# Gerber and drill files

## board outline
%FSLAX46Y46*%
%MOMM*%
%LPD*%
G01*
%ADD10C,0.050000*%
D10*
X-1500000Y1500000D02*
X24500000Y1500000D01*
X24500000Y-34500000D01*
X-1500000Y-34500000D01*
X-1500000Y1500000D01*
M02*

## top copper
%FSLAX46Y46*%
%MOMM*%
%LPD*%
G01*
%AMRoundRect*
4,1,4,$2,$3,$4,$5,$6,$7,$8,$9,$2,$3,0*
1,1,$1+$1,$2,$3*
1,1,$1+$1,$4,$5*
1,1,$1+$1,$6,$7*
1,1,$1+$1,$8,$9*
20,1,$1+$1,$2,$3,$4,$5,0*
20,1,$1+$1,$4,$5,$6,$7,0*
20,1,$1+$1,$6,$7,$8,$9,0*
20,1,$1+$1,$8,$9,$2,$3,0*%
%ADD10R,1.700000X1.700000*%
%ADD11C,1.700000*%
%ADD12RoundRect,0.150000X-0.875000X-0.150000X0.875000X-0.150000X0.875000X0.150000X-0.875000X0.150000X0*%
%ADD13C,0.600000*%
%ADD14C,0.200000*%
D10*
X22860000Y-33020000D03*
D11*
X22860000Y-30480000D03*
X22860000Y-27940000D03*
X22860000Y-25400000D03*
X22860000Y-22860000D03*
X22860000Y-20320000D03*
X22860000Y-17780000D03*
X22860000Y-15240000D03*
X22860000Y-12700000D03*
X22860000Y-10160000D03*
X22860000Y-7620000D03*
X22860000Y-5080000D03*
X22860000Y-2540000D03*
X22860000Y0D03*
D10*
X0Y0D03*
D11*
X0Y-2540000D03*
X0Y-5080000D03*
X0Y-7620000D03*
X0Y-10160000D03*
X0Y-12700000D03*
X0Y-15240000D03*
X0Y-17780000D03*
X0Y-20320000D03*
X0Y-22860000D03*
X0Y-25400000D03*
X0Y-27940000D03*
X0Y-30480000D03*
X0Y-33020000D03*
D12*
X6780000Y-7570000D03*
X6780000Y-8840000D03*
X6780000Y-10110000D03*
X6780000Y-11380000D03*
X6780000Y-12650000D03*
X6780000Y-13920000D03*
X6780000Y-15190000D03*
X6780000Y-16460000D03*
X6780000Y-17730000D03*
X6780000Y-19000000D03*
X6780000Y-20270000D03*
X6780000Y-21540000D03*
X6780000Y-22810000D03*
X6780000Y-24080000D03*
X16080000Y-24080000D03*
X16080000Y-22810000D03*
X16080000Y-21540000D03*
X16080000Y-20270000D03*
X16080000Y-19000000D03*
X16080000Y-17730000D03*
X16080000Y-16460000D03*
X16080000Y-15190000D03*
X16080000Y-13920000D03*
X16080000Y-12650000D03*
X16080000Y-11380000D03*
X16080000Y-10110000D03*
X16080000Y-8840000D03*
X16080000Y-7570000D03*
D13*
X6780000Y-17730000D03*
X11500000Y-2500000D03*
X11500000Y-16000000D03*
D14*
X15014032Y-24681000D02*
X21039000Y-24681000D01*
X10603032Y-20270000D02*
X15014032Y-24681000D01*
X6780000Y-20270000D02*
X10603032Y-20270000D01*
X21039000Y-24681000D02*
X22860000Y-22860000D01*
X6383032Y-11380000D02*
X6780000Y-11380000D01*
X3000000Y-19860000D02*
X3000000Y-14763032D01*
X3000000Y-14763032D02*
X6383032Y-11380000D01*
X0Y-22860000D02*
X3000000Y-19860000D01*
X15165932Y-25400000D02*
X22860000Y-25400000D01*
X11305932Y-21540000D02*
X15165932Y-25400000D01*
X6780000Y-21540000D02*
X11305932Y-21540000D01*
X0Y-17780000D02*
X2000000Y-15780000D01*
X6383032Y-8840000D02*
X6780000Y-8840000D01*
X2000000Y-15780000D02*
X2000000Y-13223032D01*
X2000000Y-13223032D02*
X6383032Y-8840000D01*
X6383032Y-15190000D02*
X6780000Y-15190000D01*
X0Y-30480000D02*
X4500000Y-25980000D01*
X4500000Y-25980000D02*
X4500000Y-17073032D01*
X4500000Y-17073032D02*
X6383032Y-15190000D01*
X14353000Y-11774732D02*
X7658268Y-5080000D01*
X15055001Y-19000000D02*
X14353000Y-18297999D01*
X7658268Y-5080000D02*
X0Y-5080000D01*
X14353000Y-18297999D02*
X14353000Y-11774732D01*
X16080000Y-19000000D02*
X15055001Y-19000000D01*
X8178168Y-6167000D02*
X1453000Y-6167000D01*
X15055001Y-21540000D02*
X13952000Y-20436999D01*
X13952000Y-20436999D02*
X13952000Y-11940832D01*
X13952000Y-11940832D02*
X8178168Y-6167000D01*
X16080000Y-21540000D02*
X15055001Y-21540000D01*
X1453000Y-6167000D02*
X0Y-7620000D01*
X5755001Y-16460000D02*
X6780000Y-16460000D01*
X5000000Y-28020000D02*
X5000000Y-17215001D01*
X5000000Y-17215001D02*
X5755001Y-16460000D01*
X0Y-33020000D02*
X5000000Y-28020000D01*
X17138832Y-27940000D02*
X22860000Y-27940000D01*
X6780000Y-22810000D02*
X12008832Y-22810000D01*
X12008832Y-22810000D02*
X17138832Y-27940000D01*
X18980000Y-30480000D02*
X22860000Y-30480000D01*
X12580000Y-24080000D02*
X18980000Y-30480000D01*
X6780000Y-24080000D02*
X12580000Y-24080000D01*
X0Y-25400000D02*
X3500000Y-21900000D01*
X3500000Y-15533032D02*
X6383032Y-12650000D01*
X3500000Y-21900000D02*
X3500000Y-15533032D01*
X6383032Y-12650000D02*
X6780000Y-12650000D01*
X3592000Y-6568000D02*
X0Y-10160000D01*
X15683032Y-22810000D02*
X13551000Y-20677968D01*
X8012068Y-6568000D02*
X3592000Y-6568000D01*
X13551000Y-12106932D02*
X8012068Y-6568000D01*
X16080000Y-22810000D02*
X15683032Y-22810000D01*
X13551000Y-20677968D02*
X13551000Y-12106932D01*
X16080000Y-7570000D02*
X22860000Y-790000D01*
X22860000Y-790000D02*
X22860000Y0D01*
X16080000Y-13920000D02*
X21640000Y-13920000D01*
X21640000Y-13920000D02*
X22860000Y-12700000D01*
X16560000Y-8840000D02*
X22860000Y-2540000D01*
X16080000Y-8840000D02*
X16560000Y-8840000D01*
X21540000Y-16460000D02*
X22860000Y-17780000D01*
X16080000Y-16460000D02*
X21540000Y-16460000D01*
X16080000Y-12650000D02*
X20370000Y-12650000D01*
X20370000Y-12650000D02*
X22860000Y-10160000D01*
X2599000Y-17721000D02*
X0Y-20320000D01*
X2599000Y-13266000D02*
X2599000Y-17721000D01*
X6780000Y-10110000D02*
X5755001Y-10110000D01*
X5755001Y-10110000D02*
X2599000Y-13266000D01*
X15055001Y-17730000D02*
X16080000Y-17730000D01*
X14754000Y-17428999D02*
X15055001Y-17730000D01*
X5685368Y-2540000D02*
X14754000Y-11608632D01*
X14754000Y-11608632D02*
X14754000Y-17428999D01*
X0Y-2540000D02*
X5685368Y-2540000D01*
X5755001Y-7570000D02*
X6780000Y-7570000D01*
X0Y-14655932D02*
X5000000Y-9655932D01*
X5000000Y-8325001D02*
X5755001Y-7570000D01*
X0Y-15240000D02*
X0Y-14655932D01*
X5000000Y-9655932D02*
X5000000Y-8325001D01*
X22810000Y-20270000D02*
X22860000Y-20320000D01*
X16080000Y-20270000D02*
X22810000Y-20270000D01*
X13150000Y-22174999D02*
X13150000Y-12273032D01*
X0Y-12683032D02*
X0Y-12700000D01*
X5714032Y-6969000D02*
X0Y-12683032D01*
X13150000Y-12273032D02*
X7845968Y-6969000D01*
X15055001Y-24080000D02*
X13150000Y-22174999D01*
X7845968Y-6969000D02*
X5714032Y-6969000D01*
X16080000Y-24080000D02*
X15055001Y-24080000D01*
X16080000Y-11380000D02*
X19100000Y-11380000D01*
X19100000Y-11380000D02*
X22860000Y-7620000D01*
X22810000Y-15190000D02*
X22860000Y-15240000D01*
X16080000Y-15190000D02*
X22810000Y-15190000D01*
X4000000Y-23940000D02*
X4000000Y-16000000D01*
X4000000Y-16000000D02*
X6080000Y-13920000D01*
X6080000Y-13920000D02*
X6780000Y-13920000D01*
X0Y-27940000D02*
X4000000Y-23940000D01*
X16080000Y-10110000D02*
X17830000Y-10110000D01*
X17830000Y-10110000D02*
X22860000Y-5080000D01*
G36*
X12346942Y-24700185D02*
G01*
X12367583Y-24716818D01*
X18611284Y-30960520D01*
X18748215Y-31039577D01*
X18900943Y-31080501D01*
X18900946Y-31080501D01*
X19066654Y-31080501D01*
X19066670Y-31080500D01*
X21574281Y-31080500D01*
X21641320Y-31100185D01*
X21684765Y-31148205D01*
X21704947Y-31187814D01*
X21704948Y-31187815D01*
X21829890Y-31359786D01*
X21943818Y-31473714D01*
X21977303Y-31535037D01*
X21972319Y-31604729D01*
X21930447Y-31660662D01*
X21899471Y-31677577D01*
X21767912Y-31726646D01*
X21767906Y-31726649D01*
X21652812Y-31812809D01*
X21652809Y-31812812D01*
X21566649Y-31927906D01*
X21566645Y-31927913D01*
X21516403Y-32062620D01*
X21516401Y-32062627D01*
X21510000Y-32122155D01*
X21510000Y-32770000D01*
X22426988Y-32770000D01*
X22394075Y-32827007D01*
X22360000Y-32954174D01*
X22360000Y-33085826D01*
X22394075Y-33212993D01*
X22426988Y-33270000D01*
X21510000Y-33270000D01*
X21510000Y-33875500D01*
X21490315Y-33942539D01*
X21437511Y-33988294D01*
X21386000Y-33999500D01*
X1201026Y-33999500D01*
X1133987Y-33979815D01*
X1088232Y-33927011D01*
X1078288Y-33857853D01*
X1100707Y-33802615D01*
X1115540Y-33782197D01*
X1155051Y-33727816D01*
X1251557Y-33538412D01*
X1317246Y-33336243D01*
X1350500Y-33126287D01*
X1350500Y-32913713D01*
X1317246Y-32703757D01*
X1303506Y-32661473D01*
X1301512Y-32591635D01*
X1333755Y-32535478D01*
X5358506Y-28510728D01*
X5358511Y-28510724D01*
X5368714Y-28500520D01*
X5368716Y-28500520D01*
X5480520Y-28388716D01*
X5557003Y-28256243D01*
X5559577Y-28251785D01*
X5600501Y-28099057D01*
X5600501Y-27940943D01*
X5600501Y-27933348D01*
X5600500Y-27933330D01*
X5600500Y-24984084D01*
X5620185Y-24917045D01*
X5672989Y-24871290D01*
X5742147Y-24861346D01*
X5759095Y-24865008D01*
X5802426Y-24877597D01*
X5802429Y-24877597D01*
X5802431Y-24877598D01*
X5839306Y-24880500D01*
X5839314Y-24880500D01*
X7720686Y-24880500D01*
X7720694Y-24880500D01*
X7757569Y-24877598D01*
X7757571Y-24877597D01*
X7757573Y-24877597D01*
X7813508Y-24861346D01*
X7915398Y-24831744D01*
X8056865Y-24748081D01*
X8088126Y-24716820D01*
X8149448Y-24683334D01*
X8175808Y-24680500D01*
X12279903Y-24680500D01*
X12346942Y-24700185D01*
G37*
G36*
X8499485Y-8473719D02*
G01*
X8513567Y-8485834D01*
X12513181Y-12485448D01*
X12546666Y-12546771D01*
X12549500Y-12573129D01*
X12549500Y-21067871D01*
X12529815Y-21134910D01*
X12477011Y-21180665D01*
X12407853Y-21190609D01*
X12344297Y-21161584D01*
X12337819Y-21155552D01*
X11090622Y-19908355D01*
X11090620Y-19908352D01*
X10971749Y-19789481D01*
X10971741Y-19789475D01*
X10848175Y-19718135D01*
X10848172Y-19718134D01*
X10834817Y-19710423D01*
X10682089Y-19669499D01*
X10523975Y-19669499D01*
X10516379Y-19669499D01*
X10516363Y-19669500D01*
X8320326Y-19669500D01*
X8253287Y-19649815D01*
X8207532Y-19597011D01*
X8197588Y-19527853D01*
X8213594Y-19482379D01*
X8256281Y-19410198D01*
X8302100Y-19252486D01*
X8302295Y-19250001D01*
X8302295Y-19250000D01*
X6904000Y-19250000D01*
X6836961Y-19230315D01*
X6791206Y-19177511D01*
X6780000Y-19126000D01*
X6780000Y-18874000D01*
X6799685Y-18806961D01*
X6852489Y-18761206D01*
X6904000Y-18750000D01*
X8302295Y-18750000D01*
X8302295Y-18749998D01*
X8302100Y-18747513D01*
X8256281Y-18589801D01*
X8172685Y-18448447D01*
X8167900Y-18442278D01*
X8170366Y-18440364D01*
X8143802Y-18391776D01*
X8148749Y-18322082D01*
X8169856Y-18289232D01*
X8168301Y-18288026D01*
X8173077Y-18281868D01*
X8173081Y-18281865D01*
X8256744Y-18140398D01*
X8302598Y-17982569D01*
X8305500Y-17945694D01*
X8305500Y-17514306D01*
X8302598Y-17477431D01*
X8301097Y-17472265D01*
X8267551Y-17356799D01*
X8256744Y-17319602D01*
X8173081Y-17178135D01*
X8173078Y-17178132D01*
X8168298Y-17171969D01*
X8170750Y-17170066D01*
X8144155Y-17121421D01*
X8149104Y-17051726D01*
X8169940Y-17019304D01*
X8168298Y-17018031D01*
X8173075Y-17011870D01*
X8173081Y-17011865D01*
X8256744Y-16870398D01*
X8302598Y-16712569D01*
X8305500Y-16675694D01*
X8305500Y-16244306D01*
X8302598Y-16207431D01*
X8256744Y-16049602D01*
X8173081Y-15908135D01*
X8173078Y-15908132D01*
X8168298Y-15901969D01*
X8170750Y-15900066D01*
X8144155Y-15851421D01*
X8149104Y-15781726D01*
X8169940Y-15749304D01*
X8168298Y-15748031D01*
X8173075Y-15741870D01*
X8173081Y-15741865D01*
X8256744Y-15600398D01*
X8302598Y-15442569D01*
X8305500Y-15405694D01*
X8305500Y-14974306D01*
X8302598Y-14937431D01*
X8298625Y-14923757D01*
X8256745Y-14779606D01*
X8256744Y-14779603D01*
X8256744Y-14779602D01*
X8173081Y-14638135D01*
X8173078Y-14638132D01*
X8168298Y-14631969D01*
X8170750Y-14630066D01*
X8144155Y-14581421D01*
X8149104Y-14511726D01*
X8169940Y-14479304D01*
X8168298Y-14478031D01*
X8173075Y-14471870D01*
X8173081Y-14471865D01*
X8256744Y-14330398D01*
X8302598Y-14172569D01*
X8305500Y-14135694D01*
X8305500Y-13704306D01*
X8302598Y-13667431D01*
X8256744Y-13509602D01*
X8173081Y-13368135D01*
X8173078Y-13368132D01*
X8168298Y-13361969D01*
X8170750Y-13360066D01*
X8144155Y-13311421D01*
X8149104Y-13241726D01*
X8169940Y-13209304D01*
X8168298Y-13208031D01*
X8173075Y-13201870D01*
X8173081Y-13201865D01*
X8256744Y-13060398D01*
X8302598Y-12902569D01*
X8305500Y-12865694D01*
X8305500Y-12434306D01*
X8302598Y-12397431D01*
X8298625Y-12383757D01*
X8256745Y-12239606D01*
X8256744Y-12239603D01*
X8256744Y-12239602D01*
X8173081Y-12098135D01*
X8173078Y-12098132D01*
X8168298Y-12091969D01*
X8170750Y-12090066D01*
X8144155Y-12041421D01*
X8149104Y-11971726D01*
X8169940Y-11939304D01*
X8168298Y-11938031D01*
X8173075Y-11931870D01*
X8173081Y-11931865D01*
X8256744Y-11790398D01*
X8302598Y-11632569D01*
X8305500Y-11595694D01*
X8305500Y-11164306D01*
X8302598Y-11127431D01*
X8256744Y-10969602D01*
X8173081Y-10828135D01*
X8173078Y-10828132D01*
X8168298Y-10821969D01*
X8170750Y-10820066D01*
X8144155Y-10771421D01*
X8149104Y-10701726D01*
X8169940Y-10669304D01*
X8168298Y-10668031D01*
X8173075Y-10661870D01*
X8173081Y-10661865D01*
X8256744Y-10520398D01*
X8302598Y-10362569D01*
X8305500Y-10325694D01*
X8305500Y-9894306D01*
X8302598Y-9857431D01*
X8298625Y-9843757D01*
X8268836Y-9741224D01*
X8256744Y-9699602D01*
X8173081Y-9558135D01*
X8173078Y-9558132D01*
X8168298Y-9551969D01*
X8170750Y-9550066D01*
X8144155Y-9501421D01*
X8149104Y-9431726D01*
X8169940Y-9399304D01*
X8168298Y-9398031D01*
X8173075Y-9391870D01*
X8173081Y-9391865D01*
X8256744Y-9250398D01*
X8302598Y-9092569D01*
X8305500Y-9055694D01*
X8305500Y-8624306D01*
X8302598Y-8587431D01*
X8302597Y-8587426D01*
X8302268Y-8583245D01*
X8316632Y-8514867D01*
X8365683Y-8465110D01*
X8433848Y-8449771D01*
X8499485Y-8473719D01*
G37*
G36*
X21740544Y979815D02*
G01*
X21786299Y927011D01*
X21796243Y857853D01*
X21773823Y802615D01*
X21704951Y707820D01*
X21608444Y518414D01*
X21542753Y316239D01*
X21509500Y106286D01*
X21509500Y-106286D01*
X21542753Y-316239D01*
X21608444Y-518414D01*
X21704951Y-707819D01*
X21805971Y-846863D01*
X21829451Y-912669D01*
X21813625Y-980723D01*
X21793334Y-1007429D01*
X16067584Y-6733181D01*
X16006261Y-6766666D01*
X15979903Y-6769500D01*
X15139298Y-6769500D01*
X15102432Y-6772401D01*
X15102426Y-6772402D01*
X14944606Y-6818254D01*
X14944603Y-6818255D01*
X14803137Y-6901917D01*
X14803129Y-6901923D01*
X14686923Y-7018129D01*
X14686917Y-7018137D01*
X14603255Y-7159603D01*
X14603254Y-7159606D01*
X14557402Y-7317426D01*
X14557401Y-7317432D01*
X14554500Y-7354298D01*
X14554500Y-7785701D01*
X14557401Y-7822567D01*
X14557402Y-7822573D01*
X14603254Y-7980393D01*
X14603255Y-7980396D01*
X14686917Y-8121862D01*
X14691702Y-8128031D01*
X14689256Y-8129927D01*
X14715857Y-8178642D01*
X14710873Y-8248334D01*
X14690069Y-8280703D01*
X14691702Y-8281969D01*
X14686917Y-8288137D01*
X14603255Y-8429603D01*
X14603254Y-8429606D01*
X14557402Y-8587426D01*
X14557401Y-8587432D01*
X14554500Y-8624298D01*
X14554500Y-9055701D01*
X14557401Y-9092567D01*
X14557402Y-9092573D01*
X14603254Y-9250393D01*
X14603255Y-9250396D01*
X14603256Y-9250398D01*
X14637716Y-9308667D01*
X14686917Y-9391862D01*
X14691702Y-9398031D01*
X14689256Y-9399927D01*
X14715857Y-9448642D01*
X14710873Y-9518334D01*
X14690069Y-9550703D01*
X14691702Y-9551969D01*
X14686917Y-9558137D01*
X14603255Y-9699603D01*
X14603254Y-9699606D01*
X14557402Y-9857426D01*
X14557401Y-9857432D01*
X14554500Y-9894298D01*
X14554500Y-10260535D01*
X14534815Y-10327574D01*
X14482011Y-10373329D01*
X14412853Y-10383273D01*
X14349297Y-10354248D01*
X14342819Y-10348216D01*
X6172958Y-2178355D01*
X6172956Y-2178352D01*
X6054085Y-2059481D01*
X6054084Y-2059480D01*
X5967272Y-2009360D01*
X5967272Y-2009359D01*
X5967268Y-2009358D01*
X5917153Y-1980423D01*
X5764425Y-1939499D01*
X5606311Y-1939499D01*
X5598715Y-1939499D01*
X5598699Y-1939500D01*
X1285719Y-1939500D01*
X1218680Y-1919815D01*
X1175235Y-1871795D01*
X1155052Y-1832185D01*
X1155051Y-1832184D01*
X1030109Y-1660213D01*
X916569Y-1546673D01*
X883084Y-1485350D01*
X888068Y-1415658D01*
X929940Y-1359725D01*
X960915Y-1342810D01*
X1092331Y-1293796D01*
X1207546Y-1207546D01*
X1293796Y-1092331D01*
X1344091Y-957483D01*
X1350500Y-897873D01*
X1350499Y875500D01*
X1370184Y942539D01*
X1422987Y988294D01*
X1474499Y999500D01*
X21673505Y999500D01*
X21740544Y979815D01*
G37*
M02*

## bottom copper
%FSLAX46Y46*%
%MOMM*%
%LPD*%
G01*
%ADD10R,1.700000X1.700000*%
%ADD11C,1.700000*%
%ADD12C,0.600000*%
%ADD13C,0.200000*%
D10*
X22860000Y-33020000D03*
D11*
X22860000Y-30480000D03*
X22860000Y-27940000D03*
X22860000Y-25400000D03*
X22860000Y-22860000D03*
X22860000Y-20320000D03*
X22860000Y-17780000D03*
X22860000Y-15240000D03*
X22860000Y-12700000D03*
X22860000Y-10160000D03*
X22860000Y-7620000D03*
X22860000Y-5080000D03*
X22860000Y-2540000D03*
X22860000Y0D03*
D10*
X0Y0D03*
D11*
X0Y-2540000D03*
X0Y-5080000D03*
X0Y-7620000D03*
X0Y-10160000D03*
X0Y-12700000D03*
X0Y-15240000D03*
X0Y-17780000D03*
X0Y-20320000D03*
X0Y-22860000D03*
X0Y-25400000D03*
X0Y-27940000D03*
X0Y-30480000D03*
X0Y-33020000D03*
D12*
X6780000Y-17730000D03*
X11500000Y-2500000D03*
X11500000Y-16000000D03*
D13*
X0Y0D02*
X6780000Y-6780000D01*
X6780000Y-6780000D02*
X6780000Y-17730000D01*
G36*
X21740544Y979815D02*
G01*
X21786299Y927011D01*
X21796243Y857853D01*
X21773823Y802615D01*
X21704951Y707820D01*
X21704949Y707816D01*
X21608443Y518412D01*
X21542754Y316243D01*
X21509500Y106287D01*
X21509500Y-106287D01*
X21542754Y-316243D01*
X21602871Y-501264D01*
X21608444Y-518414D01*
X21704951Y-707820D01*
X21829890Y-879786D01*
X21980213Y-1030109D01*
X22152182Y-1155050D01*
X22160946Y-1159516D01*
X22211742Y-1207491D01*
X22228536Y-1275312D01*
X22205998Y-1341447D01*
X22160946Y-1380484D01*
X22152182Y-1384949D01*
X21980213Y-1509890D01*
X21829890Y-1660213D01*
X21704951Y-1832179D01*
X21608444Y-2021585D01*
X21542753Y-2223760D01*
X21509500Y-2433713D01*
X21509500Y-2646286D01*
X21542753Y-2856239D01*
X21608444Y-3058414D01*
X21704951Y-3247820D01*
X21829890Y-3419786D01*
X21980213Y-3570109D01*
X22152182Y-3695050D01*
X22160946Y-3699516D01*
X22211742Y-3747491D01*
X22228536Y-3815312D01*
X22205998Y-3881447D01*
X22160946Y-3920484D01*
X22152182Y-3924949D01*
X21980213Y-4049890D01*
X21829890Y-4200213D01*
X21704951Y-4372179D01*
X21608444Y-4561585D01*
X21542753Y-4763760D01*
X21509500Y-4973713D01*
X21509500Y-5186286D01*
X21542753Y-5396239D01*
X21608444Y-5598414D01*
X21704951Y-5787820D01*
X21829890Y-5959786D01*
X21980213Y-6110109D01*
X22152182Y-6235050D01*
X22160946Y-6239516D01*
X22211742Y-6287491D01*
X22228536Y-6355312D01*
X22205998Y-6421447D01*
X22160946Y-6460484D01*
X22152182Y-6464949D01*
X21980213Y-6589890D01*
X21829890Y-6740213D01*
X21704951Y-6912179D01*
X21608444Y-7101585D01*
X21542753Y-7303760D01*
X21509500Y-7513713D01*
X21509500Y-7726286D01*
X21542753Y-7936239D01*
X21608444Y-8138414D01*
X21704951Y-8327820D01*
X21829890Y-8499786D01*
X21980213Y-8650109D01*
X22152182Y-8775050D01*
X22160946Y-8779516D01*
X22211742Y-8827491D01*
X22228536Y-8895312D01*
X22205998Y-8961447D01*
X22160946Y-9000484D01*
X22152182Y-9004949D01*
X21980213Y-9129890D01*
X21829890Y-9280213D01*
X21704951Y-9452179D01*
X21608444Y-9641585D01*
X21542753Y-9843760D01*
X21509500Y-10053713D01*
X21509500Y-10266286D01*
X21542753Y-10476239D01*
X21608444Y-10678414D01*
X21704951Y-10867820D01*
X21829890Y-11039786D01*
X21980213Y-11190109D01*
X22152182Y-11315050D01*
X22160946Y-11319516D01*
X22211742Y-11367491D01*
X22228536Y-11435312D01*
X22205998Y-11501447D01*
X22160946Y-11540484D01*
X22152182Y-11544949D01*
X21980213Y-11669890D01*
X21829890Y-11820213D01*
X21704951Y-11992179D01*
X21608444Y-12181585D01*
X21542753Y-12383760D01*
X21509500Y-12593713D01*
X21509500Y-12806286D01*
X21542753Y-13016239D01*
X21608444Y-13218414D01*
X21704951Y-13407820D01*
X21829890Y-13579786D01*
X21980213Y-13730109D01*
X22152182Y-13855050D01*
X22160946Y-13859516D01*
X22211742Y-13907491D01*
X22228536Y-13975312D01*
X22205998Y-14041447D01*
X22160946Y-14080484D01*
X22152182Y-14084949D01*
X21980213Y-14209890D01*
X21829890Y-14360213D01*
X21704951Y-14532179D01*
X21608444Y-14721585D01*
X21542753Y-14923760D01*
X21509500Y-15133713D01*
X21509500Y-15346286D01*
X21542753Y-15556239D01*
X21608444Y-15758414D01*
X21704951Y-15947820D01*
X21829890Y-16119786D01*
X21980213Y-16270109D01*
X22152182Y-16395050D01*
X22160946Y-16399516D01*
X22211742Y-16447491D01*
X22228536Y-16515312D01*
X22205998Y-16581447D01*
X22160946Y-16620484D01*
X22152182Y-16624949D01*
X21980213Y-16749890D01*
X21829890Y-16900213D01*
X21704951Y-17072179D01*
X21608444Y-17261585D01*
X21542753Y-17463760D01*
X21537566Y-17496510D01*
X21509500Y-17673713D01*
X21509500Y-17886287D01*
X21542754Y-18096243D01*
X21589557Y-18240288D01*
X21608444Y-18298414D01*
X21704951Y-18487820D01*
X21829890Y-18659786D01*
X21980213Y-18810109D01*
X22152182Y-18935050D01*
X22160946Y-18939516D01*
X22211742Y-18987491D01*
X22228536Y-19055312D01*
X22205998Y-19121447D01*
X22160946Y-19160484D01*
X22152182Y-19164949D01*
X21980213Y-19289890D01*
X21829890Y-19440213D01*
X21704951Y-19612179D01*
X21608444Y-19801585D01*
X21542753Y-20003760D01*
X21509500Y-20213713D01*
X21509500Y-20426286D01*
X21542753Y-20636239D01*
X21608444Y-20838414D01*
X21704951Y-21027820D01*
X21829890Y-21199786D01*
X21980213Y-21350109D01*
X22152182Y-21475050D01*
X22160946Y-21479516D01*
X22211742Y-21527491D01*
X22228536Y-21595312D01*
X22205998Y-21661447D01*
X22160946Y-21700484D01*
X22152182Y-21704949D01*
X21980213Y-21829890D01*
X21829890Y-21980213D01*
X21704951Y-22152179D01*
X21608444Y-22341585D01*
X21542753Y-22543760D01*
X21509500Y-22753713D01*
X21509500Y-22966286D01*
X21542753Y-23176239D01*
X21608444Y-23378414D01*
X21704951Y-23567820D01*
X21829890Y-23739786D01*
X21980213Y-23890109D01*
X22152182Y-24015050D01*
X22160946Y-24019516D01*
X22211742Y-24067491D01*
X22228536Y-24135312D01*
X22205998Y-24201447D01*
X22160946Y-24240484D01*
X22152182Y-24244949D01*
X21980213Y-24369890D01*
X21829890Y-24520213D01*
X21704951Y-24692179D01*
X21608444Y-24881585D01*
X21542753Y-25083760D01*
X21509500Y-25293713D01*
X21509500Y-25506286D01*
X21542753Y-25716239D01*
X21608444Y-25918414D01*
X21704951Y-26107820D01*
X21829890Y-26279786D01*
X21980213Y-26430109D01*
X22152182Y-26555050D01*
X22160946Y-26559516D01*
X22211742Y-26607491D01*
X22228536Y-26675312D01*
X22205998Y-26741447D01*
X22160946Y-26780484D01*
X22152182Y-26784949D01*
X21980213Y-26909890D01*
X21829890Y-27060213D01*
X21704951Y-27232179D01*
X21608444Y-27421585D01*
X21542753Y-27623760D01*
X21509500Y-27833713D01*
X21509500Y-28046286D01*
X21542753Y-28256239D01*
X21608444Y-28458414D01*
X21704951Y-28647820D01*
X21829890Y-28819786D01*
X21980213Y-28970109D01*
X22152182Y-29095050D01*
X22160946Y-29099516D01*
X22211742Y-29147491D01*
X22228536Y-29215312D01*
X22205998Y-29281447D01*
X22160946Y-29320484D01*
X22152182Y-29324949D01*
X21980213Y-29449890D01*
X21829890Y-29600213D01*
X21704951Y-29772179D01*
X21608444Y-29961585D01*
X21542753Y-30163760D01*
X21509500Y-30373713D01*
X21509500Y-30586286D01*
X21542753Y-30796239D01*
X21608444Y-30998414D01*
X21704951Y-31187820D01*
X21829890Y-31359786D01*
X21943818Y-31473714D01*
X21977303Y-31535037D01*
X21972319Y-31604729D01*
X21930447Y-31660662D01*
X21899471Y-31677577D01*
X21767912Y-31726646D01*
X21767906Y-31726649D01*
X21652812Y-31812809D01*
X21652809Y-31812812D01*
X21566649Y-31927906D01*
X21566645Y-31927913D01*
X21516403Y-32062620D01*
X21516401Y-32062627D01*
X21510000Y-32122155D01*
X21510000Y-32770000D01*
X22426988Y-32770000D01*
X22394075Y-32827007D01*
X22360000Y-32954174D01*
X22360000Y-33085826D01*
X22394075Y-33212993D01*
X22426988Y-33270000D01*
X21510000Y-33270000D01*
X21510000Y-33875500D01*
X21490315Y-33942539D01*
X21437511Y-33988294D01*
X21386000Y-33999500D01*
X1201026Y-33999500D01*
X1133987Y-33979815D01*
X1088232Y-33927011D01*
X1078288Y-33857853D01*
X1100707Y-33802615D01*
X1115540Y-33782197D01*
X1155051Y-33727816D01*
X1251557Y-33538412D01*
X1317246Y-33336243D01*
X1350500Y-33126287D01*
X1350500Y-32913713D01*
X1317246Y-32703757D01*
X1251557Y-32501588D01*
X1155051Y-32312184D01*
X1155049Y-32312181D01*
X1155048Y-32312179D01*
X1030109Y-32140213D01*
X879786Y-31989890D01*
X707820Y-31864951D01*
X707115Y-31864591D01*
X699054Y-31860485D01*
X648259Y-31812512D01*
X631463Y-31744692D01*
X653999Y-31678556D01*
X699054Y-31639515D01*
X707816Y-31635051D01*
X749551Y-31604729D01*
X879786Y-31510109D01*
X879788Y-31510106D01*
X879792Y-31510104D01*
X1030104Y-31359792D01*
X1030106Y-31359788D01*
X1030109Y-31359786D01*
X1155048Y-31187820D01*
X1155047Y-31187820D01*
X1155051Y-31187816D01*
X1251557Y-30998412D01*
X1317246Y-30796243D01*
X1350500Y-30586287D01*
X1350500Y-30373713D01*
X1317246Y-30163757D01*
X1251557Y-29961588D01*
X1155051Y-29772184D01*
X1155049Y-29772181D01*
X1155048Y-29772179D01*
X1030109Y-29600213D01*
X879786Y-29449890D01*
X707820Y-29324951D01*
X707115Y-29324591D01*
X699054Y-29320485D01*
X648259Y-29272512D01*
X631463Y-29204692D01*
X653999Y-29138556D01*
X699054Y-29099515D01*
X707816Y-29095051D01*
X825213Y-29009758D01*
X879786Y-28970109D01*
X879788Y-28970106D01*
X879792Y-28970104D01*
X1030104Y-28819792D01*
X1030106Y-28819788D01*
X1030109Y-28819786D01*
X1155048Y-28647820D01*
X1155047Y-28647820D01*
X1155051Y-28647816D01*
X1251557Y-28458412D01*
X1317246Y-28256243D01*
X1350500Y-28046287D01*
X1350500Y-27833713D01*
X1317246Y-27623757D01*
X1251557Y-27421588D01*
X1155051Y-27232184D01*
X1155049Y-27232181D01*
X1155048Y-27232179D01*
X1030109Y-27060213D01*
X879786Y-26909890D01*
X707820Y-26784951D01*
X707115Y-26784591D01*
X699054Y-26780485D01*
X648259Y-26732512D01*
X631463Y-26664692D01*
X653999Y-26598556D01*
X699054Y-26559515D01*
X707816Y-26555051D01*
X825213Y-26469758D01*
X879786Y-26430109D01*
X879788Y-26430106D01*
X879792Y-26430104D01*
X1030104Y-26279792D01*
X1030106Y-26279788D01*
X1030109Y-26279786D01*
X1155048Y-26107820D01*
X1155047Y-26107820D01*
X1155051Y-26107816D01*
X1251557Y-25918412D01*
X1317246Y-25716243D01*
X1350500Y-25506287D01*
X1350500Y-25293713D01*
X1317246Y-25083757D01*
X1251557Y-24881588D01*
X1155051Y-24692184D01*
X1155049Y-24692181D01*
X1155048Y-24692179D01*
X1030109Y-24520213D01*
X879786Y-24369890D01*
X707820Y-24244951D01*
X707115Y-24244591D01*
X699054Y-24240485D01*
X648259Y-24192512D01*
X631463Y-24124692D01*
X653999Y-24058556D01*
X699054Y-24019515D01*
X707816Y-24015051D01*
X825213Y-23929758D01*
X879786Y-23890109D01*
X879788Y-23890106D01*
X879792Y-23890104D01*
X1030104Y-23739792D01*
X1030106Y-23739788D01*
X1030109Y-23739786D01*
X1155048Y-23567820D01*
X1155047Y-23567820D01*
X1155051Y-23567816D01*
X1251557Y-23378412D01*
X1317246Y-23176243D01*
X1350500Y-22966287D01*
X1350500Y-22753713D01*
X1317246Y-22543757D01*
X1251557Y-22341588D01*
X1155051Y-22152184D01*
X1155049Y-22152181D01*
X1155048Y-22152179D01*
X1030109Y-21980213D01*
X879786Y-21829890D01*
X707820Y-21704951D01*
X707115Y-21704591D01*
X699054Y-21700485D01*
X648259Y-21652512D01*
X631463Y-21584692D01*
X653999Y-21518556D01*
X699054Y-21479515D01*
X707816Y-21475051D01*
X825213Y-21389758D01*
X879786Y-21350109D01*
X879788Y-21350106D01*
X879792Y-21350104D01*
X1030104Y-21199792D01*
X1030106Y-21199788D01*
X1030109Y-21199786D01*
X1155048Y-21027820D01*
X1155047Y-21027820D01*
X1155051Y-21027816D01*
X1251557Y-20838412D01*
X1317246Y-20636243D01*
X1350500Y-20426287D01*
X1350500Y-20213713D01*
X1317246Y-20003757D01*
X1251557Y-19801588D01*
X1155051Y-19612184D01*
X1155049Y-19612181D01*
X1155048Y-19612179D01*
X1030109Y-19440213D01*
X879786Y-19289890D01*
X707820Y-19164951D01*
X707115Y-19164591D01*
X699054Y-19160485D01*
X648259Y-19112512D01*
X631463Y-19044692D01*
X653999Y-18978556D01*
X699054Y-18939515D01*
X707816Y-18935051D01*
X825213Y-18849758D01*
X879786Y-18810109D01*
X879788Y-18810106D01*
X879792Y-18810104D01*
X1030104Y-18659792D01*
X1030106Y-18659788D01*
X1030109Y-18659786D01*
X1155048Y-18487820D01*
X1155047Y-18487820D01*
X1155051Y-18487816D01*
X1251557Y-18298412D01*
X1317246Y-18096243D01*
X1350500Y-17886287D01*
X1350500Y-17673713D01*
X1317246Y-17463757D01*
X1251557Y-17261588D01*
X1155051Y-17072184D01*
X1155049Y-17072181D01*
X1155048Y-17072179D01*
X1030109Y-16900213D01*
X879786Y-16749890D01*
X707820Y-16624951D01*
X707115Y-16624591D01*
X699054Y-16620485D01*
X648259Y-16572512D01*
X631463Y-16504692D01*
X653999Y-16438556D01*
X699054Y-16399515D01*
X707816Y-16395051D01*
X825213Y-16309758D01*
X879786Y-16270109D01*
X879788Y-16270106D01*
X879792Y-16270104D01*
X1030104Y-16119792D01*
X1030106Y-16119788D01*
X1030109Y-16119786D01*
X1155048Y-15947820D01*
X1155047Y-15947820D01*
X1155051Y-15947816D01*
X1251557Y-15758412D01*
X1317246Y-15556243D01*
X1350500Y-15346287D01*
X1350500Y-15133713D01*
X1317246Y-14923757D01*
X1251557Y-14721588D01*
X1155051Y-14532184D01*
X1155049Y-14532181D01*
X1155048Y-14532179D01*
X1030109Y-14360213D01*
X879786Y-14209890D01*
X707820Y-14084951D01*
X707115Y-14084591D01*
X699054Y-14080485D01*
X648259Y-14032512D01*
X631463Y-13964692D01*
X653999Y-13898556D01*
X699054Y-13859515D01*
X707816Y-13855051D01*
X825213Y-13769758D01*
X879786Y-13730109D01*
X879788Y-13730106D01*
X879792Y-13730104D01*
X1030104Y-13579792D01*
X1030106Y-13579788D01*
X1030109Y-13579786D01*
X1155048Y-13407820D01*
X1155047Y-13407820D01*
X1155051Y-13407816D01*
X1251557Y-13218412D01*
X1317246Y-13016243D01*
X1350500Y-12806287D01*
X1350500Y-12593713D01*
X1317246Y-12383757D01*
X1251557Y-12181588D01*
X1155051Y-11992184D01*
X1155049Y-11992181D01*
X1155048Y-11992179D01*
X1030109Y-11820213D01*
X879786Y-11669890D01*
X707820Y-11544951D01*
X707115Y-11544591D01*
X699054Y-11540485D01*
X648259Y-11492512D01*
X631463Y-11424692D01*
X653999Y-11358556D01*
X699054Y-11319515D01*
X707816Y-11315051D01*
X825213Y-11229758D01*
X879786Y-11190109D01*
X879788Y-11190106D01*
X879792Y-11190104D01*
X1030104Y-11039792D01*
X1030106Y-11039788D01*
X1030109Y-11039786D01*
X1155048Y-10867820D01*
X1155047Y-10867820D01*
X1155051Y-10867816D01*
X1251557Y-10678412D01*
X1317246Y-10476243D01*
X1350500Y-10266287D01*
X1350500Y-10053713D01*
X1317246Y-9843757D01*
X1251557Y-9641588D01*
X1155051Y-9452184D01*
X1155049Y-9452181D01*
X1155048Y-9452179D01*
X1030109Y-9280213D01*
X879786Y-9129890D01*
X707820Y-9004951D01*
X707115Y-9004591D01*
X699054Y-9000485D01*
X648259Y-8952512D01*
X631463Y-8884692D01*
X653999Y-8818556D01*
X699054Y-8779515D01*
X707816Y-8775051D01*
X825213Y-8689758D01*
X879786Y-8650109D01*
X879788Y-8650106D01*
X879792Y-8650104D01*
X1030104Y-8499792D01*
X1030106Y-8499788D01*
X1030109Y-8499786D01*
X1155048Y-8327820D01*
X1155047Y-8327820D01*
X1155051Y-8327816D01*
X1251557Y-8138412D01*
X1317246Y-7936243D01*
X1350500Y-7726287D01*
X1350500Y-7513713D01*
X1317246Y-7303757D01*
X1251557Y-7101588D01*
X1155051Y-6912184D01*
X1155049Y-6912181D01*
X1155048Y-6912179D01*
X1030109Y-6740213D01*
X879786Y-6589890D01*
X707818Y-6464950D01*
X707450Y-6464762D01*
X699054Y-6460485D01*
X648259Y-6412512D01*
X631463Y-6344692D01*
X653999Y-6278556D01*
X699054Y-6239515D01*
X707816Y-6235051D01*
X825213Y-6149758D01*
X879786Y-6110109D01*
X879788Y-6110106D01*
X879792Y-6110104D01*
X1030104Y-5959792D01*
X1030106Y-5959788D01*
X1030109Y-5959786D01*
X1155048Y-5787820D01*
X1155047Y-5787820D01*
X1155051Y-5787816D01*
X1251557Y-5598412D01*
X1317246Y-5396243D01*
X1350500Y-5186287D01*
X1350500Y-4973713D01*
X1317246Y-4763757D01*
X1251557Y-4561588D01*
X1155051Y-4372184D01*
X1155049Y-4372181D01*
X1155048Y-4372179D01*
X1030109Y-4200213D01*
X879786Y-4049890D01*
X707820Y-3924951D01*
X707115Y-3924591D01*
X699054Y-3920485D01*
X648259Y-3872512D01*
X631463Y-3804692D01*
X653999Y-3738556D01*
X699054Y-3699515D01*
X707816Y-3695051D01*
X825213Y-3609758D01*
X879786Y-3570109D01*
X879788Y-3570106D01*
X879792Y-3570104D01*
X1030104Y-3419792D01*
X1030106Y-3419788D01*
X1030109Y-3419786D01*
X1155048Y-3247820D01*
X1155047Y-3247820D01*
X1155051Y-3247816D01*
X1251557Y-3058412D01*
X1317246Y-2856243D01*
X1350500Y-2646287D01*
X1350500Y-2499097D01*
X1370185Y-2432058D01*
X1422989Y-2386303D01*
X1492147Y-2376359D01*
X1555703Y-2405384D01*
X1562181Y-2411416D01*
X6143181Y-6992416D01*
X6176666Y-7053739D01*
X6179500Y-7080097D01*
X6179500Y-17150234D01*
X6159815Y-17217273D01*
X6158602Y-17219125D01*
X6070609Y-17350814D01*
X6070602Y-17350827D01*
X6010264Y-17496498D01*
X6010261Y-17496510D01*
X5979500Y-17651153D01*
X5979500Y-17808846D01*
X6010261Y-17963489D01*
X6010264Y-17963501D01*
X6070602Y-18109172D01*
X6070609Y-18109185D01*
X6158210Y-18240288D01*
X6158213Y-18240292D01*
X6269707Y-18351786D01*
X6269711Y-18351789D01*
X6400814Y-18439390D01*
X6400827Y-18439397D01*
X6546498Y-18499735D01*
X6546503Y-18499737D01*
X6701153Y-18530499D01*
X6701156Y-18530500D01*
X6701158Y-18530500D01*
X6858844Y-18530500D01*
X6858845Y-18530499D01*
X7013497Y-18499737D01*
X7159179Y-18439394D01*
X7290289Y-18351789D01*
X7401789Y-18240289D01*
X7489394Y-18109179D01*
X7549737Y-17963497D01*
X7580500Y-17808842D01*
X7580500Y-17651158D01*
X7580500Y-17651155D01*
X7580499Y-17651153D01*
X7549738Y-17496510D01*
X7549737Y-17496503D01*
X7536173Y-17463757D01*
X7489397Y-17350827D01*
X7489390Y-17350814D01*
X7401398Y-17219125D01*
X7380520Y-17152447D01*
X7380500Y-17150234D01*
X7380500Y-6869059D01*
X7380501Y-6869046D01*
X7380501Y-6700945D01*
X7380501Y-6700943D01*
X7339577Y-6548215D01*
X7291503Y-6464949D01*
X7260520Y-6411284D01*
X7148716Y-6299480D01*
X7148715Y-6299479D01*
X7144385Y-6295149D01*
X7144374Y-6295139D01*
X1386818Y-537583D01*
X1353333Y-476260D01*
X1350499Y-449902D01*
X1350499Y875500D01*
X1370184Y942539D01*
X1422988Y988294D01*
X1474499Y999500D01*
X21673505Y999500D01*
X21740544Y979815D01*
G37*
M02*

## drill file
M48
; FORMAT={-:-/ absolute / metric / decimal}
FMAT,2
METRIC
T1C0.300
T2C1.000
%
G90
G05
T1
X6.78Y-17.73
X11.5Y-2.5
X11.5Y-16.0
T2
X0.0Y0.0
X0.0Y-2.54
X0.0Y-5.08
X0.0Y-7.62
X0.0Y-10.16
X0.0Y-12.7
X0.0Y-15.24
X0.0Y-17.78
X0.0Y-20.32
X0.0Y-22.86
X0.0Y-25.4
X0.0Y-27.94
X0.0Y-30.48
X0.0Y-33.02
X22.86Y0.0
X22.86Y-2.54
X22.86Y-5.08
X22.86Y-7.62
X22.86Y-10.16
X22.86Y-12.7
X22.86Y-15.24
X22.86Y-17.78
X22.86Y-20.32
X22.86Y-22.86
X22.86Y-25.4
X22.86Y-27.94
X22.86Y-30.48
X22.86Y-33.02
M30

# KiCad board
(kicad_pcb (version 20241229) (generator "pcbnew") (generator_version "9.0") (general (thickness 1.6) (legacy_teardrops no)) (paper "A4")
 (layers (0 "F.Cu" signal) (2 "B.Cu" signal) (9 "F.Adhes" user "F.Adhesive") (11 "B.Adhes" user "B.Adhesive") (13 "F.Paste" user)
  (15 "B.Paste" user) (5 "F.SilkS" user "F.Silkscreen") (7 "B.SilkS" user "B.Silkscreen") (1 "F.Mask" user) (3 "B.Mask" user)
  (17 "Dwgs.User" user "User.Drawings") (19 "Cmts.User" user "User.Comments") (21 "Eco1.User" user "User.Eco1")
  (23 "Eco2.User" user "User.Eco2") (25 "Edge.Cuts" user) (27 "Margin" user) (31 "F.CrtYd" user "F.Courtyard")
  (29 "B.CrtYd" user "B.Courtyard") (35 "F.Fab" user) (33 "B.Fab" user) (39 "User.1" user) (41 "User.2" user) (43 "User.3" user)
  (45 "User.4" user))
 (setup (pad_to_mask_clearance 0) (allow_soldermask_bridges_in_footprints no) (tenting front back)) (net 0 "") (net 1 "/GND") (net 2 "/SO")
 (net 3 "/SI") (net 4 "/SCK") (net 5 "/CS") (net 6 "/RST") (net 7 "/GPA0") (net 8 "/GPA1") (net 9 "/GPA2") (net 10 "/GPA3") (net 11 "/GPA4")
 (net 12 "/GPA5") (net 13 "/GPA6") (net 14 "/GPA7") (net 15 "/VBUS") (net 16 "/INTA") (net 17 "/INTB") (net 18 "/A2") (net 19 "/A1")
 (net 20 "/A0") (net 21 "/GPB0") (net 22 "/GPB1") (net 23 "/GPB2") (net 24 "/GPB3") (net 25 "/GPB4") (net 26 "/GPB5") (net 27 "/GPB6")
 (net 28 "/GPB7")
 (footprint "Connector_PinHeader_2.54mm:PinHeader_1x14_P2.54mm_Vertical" (layer "F.Cu") (at 22.86 33.02 180)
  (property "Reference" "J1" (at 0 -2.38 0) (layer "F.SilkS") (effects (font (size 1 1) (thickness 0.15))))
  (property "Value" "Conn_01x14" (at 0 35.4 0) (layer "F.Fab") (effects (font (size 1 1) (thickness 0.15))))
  (pad "1" thru_hole rect (at 0 0 180) (size 1.7 1.7) (drill 1) (layers "*.Cu" "*.Mask") (remove_unused_layers no) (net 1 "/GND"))
  (pad "2" thru_hole circle (at 0 2.54 180) (size 1.7 1.7) (drill 1) (layers "*.Cu" "*.Mask") (remove_unused_layers no) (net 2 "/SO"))
  (pad "3" thru_hole circle (at 0 5.08 180) (size 1.7 1.7) (drill 1) (layers "*.Cu" "*.Mask") (remove_unused_layers no) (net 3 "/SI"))
  (pad "4" thru_hole circle (at 0 7.62 180) (size 1.7 1.7) (drill 1) (layers "*.Cu" "*.Mask") (remove_unused_layers no) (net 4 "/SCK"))
  (pad "5" thru_hole circle (at 0 10.16 180) (size 1.7 1.7) (drill 1) (layers "*.Cu" "*.Mask") (remove_unused_layers no) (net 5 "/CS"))
  (pad "6" thru_hole circle (at 0 12.7 180) (size 1.7 1.7) (drill 1) (layers "*.Cu" "*.Mask") (remove_unused_layers no) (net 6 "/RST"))
  (pad "7" thru_hole circle (at 0 15.24 180) (size 1.7 1.7) (drill 1) (layers "*.Cu" "*.Mask") (remove_unused_layers no) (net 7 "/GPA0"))
  (pad "8" thru_hole circle (at 0 17.78 180) (size 1.7 1.7) (drill 1) (layers "*.Cu" "*.Mask") (remove_unused_layers no) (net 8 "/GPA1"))
  (pad "9" thru_hole circle (at 0 20.32 180) (size 1.7 1.7) (drill 1) (layers "*.Cu" "*.Mask") (remove_unused_layers no) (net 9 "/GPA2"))
  (pad "10" thru_hole circle (at 0 22.86 180) (size 1.7 1.7) (drill 1) (layers "*.Cu" "*.Mask") (remove_unused_layers no) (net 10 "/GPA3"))
  (pad "11" thru_hole circle (at 0 25.4 180) (size 1.7 1.7) (drill 1) (layers "*.Cu" "*.Mask") (remove_unused_layers no) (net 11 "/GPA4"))
  (pad "12" thru_hole circle (at 0 27.94 180) (size 1.7 1.7) (drill 1) (layers "*.Cu" "*.Mask") (remove_unused_layers no) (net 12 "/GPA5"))
  (pad "13" thru_hole circle (at 0 30.48 180) (size 1.7 1.7) (drill 1) (layers "*.Cu" "*.Mask") (remove_unused_layers no) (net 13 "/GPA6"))
  (pad "14" thru_hole circle (at 0 33.02 180) (size 1.7 1.7) (drill 1) (layers "*.Cu" "*.Mask") (remove_unused_layers no) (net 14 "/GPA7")))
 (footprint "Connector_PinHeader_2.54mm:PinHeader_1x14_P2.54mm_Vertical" (layer "F.Cu") (at 0 0)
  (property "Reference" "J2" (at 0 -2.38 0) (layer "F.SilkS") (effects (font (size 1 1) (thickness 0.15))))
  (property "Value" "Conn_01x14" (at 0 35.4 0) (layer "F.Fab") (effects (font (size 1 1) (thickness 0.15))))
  (pad "1" thru_hole rect (at 0 0) (size 1.7 1.7) (drill 1) (layers "*.Cu" "*.Mask") (remove_unused_layers no) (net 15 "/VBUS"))
  (pad "2" thru_hole circle (at 0 2.54) (size 1.7 1.7) (drill 1) (layers "*.Cu" "*.Mask") (remove_unused_layers no) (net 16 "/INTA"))
  (pad "3" thru_hole circle (at 0 5.08) (size 1.7 1.7) (drill 1) (layers "*.Cu" "*.Mask") (remove_unused_layers no) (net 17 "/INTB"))
  (pad "4" thru_hole circle (at 0 7.62) (size 1.7 1.7) (drill 1) (layers "*.Cu" "*.Mask") (remove_unused_layers no) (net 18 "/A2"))
  (pad "5" thru_hole circle (at 0 10.16) (size 1.7 1.7) (drill 1) (layers "*.Cu" "*.Mask") (remove_unused_layers no) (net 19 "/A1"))
  (pad "6" thru_hole circle (at 0 12.7) (size 1.7 1.7) (drill 1) (layers "*.Cu" "*.Mask") (remove_unused_layers no) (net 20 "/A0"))
  (pad "7" thru_hole circle (at 0 15.24) (size 1.7 1.7) (drill 1) (layers "*.Cu" "*.Mask") (remove_unused_layers no) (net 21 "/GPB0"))
  (pad "8" thru_hole circle (at 0 17.78) (size 1.7 1.7) (drill 1) (layers "*.Cu" "*.Mask") (remove_unused_layers no) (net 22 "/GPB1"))
  (pad "9" thru_hole circle (at 0 20.32) (size 1.7 1.7) (drill 1) (layers "*.Cu" "*.Mask") (remove_unused_layers no) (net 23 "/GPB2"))
  (pad "10" thru_hole circle (at 0 22.86) (size 1.7 1.7) (drill 1) (layers "*.Cu" "*.Mask") (remove_unused_layers no) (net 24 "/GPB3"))
  (pad "11" thru_hole circle (at 0 25.4) (size 1.7 1.7) (drill 1) (layers "*.Cu" "*.Mask") (remove_unused_layers no) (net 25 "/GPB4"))
  (pad "12" thru_hole circle (at 0 27.94) (size 1.7 1.7) (drill 1) (layers "*.Cu" "*.Mask") (remove_unused_layers no) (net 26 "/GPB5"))
  (pad "13" thru_hole circle (at 0 30.48) (size 1.7 1.7) (drill 1) (layers "*.Cu" "*.Mask") (remove_unused_layers no) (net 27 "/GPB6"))
  (pad "14" thru_hole circle (at 0 33.02) (size 1.7 1.7) (drill 1) (layers "*.Cu" "*.Mask") (remove_unused_layers no) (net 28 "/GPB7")))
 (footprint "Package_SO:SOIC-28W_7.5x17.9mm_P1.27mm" (layer "F.Cu") (at 11.43 15.825)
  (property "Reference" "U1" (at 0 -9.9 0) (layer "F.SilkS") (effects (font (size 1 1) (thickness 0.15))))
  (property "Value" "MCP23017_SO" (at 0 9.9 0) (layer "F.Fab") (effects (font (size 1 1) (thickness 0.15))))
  (pad "1" smd roundrect (at -4.65 -8.255) (size 2.05 0.6) (layers "F.Cu" "F.Mask" "F.Paste") (roundrect_rratio 0.25) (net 21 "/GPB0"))
  (pad "2" smd roundrect (at -4.65 -6.985) (size 2.05 0.6) (layers "F.Cu" "F.Mask" "F.Paste") (roundrect_rratio 0.25) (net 22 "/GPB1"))
  (pad "3" smd roundrect (at -4.65 -5.715) (size 2.05 0.6) (layers "F.Cu" "F.Mask" "F.Paste") (roundrect_rratio 0.25) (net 23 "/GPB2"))
  (pad "4" smd roundrect (at -4.65 -4.445) (size 2.05 0.6) (layers "F.Cu" "F.Mask" "F.Paste") (roundrect_rratio 0.25) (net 24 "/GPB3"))
  (pad "5" smd roundrect (at -4.65 -3.175) (size 2.05 0.6) (layers "F.Cu" "F.Mask" "F.Paste") (roundrect_rratio 0.25) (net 25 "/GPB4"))
  (pad "6" smd roundrect (at -4.65 -1.905) (size 2.05 0.6) (layers "F.Cu" "F.Mask" "F.Paste") (roundrect_rratio 0.25) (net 26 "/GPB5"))
  (pad "7" smd roundrect (at -4.65 -0.635) (size 2.05 0.6) (layers "F.Cu" "F.Mask" "F.Paste") (roundrect_rratio 0.25) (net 27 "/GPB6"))
  (pad "8" smd roundrect (at -4.65 0.635) (size 2.05 0.6) (layers "F.Cu" "F.Mask" "F.Paste") (roundrect_rratio 0.25) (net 28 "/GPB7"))
  (pad "9" smd roundrect (at -4.65 1.905) (size 2.05 0.6) (layers "F.Cu" "F.Mask" "F.Paste") (roundrect_rratio 0.25) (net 15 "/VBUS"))
  (pad "10" smd roundrect (at -4.65 3.175) (size 2.05 0.6) (layers "F.Cu" "F.Mask" "F.Paste") (roundrect_rratio 0.25) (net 1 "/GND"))
  (pad "11" smd roundrect (at -4.65 4.445) (size 2.05 0.6) (layers "F.Cu" "F.Mask" "F.Paste") (roundrect_rratio 0.25) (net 5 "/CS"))
  (pad "12" smd roundrect (at -4.65 5.715) (size 2.05 0.6) (layers "F.Cu" "F.Mask" "F.Paste") (roundrect_rratio 0.25) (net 4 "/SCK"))
  (pad "13" smd roundrect (at -4.65 6.985) (size 2.05 0.6) (layers "F.Cu" "F.Mask" "F.Paste") (roundrect_rratio 0.25) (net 3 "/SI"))
  (pad "14" smd roundrect (at -4.65 8.255) (size 2.05 0.6) (layers "F.Cu" "F.Mask" "F.Paste") (roundrect_rratio 0.25) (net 2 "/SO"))
  (pad "15" smd roundrect (at 4.65 8.255) (size 2.05 0.6) (layers "F.Cu" "F.Mask" "F.Paste") (roundrect_rratio 0.25) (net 20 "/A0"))
  (pad "16" smd roundrect (at 4.65 6.985) (size 2.05 0.6) (layers "F.Cu" "F.Mask" "F.Paste") (roundrect_rratio 0.25) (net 19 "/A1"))
  (pad "17" smd roundrect (at 4.65 5.715) (size 2.05 0.6) (layers "F.Cu" "F.Mask" "F.Paste") (roundrect_rratio 0.25) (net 18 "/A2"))
  (pad "18" smd roundrect (at 4.65 4.445) (size 2.05 0.6) (layers "F.Cu" "F.Mask" "F.Paste") (roundrect_rratio 0.25) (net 6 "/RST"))
  (pad "19" smd roundrect (at 4.65 3.175) (size 2.05 0.6) (layers "F.Cu" "F.Mask" "F.Paste") (roundrect_rratio 0.25) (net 17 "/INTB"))
  (pad "20" smd roundrect (at 4.65 1.905) (size 2.05 0.6) (layers "F.Cu" "F.Mask" "F.Paste") (roundrect_rratio 0.25) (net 16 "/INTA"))
  (pad "21" smd roundrect (at 4.65 0.635) (size 2.05 0.6) (layers "F.Cu" "F.Mask" "F.Paste") (roundrect_rratio 0.25) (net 7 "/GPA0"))
  (pad "22" smd roundrect (at 4.65 -0.635) (size 2.05 0.6) (layers "F.Cu" "F.Mask" "F.Paste") (roundrect_rratio 0.25) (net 8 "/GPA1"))
  (pad "23" smd roundrect (at 4.65 -1.905) (size 2.05 0.6) (layers "F.Cu" "F.Mask" "F.Paste") (roundrect_rratio 0.25) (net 9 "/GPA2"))
  (pad "24" smd roundrect (at 4.65 -3.175) (size 2.05 0.6) (layers "F.Cu" "F.Mask" "F.Paste") (roundrect_rratio 0.25) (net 10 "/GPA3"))
  (pad "25" smd roundrect (at 4.65 -4.445) (size 2.05 0.6) (layers "F.Cu" "F.Mask" "F.Paste") (roundrect_rratio 0.25) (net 11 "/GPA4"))
  (pad "26" smd roundrect (at 4.65 -5.715) (size 2.05 0.6) (layers "F.Cu" "F.Mask" "F.Paste") (roundrect_rratio 0.25) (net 12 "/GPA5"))
  (pad "27" smd roundrect (at 4.65 -6.985) (size 2.05 0.6) (layers "F.Cu" "F.Mask" "F.Paste") (roundrect_rratio 0.25) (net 13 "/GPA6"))
  (pad "28" smd roundrect (at 4.65 -8.255) (size 2.05 0.6) (layers "F.Cu" "F.Mask" "F.Paste") (roundrect_rratio 0.25) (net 14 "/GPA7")))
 (gr_rect (start -1.5 -1.5) (end 24.5 34.5) (stroke (width 0.05) (type default)) (fill no) (layer "Edge.Cuts"))
 (segment (start 15.014032 24.681) (end 21.039 24.681) (width 0.2) (layer "F.Cu") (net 5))
 (segment (start 10.603032 20.27) (end 15.014032 24.681) (width 0.2) (layer "F.Cu") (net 5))
 (segment (start 6.78 20.27) (end 10.603032 20.27) (width 0.2) (layer "F.Cu") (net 5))
 (segment (start 21.039 24.681) (end 22.86 22.86) (width 0.2) (layer "F.Cu") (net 5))
 (segment (start 6.383032 11.38) (end 6.78 11.38) (width 0.2) (layer "F.Cu") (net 24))
 (segment (start 3 19.86) (end 3 14.763032) (width 0.2) (layer "F.Cu") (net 24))
 (segment (start 3 14.763032) (end 6.383032 11.38) (width 0.2) (layer "F.Cu") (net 24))
 (segment (start 0 22.86) (end 3 19.86) (width 0.2) (layer "F.Cu") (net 24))
 (segment (start 15.165932 25.4) (end 22.86 25.4) (width 0.2) (layer "F.Cu") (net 4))
 (segment (start 11.305932 21.54) (end 15.165932 25.4) (width 0.2) (layer "F.Cu") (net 4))
 (segment (start 6.78 21.54) (end 11.305932 21.54) (width 0.2) (layer "F.Cu") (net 4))
 (segment (start 0 17.78) (end 2 15.78) (width 0.2) (layer "F.Cu") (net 22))
 (segment (start 6.383032 8.84) (end 6.78 8.84) (width 0.2) (layer "F.Cu") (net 22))
 (segment (start 2 15.78) (end 2 13.223032) (width 0.2) (layer "F.Cu") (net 22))
 (segment (start 2 13.223032) (end 6.383032 8.84) (width 0.2) (layer "F.Cu") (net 22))
 (segment (start 6.383032 15.19) (end 6.78 15.19) (width 0.2) (layer "F.Cu") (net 27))
 (segment (start 0 30.48) (end 4.5 25.98) (width 0.2) (layer "F.Cu") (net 27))
 (segment (start 4.5 25.98) (end 4.5 17.073032) (width 0.2) (layer "F.Cu") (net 27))
 (segment (start 4.5 17.073032) (end 6.383032 15.19) (width 0.2) (layer "F.Cu") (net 27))
 (via (at 6.78 17.73) (size 0.6) (drill 0.3) (layers "F.Cu" "B.Cu") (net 15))
 (segment (start 0 0) (end 6.78 6.78) (width 0.2) (layer "B.Cu") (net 15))
 (segment (start 6.78 6.78) (end 6.78 17.73) (width 0.2) (layer "B.Cu") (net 15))
 (segment (start 14.353 11.774732) (end 7.658268 5.08) (width 0.2) (layer "F.Cu") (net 17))
 (segment (start 15.055001 19) (end 14.353 18.297999) (width 0.2) (layer "F.Cu") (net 17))
 (segment (start 7.658268 5.08) (end 0 5.08) (width 0.2) (layer "F.Cu") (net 17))
 (segment (start 14.353 18.297999) (end 14.353 11.774732) (width 0.2) (layer "F.Cu") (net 17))
 (segment (start 16.08 19) (end 15.055001 19) (width 0.2) (layer "F.Cu") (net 17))
 (segment (start 8.178168 6.167) (end 1.453 6.167) (width 0.2) (layer "F.Cu") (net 18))
 (segment (start 15.055001 21.54) (end 13.952 20.436999) (width 0.2) (layer "F.Cu") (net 18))
 (segment (start 13.952 20.436999) (end 13.952 11.940832) (width 0.2) (layer "F.Cu") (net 18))
 (segment (start 13.952 11.940832) (end 8.178168 6.167) (width 0.2) (layer "F.Cu") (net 18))
 (segment (start 16.08 21.54) (end 15.055001 21.54) (width 0.2) (layer "F.Cu") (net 18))
 (segment (start 1.453 6.167) (end 0 7.62) (width 0.2) (layer "F.Cu") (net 18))
 (segment (start 5.755001 16.46) (end 6.78 16.46) (width 0.2) (layer "F.Cu") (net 28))
 (segment (start 5 28.02) (end 5 17.215001) (width 0.2) (layer "F.Cu") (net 28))
 (segment (start 5 17.215001) (end 5.755001 16.46) (width 0.2) (layer "F.Cu") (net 28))
 (segment (start 0 33.02) (end 5 28.02) (width 0.2) (layer "F.Cu") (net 28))
 (segment (start 17.138832 27.94) (end 22.86 27.94) (width 0.2) (layer "F.Cu") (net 3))
 (segment (start 6.78 22.81) (end 12.008832 22.81) (width 0.2) (layer "F.Cu") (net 3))
 (segment (start 12.008832 22.81) (end 17.138832 27.94) (width 0.2) (layer "F.Cu") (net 3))
 (segment (start 18.98 30.48) (end 22.86 30.48) (width 0.2) (layer "F.Cu") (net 2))
 (segment (start 12.58 24.08) (end 18.98 30.48) (width 0.2) (layer "F.Cu") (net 2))
 (segment (start 6.78 24.08) (end 12.58 24.08) (width 0.2) (layer "F.Cu") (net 2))
 (via (at 11.5 2.5) (size 0.6) (drill 0.3) (layers "F.Cu" "B.Cu") (free yes) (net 1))
 (via (at 11.5 16) (size 0.6) (drill 0.3) (layers "F.Cu" "B.Cu") (free yes) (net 1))
 (segment (start 0 25.4) (end 3.5 21.9) (width 0.2) (layer "F.Cu") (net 25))
 (segment (start 3.5 15.533032) (end 6.383032 12.65) (width 0.2) (layer "F.Cu") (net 25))
 (segment (start 3.5 21.9) (end 3.5 15.533032) (width 0.2) (layer "F.Cu") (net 25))
 (segment (start 6.383032 12.65) (end 6.78 12.65) (width 0.2) (layer "F.Cu") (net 25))
 (segment (start 3.592 6.568) (end 0 10.16) (width 0.2) (layer "F.Cu") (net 19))
 (segment (start 15.683032 22.81) (end 13.551 20.677968) (width 0.2) (layer "F.Cu") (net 19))
 (segment (start 8.012068 6.568) (end 3.592 6.568) (width 0.2) (layer "F.Cu") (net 19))
 (segment (start 13.551 12.106932) (end 8.012068 6.568) (width 0.2) (layer "F.Cu") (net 19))
 (segment (start 16.08 22.81) (end 15.683032 22.81) (width 0.2) (layer "F.Cu") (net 19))
 (segment (start 13.551 20.677968) (end 13.551 12.106932) (width 0.2) (layer "F.Cu") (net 19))
 (segment (start 16.08 7.57) (end 22.86 0.79) (width 0.2) (layer "F.Cu") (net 14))
 (segment (start 22.86 0.79) (end 22.86 0) (width 0.2) (layer "F.Cu") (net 14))
 (segment (start 16.08 13.92) (end 21.64 13.92) (width 0.2) (layer "F.Cu") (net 9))
 (segment (start 21.64 13.92) (end 22.86 12.7) (width 0.2) (layer "F.Cu") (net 9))
 (segment (start 16.56 8.84) (end 22.86 2.54) (width 0.2) (layer "F.Cu") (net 13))
 (segment (start 16.08 8.84) (end 16.56 8.84) (width 0.2) (layer "F.Cu") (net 13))
 (segment (start 21.54 16.46) (end 22.86 17.78) (width 0.2) (layer "F.Cu") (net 7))
 (segment (start 16.08 16.46) (end 21.54 16.46) (width 0.2) (layer "F.Cu") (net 7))
 (segment (start 16.08 12.65) (end 20.37 12.65) (width 0.2) (layer "F.Cu") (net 10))
 (segment (start 20.37 12.65) (end 22.86 10.16) (width 0.2) (layer "F.Cu") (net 10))
 (segment (start 2.599 17.721) (end 0 20.32) (width 0.2) (layer "F.Cu") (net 23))
 (segment (start 2.599 13.266) (end 2.599 17.721) (width 0.2) (layer "F.Cu") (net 23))
 (segment (start 6.78 10.11) (end 5.755001 10.11) (width 0.2) (layer "F.Cu") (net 23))
 (segment (start 5.755001 10.11) (end 2.599 13.266) (width 0.2) (layer "F.Cu") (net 23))
 (segment (start 15.055001 17.73) (end 16.08 17.73) (width 0.2) (layer "F.Cu") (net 16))
 (segment (start 14.754 17.428999) (end 15.055001 17.73) (width 0.2) (layer "F.Cu") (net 16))
 (segment (start 5.685368 2.54) (end 14.754 11.608632) (width 0.2) (layer "F.Cu") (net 16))
 (segment (start 14.754 11.608632) (end 14.754 17.428999) (width 0.2) (layer "F.Cu") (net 16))
 (segment (start 0 2.54) (end 5.685368 2.54) (width 0.2) (layer "F.Cu") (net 16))
 (segment (start 5.755001 7.57) (end 6.78 7.57) (width 0.2) (layer "F.Cu") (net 21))
 (segment (start 0 14.655932) (end 5 9.655932) (width 0.2) (layer "F.Cu") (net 21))
 (segment (start 5 8.325001) (end 5.755001 7.57) (width 0.2) (layer "F.Cu") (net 21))
 (segment (start 0 15.24) (end 0 14.655932) (width 0.2) (layer "F.Cu") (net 21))
 (segment (start 5 9.655932) (end 5 8.325001) (width 0.2) (layer "F.Cu") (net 21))
 (segment (start 22.81 20.27) (end 22.86 20.32) (width 0.2) (layer "F.Cu") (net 6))
 (segment (start 16.08 20.27) (end 22.81 20.27) (width 0.2) (layer "F.Cu") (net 6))
 (segment (start 13.15 22.174999) (end 13.15 12.273032) (width 0.2) (layer "F.Cu") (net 20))
 (segment (start 0 12.683032) (end 0 12.7) (width 0.2) (layer "F.Cu") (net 20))
 (segment (start 5.714032 6.969) (end 0 12.683032) (width 0.2) (layer "F.Cu") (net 20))
 (segment (start 13.15 12.273032) (end 7.845968 6.969) (width 0.2) (layer "F.Cu") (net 20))
 (segment (start 15.055001 24.08) (end 13.15 22.174999) (width 0.2) (layer "F.Cu") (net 20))
 (segment (start 7.845968 6.969) (end 5.714032 6.969) (width 0.2) (layer "F.Cu") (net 20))
 (segment (start 16.08 24.08) (end 15.055001 24.08) (width 0.2) (layer "F.Cu") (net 20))
 (segment (start 16.08 11.38) (end 19.1 11.38) (width 0.2) (layer "F.Cu") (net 11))
 (segment (start 19.1 11.38) (end 22.86 7.62) (width 0.2) (layer "F.Cu") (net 11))
 (segment (start 22.81 15.19) (end 22.86 15.24) (width 0.2) (layer "F.Cu") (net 8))
 (segment (start 16.08 15.19) (end 22.81 15.19) (width 0.2) (layer "F.Cu") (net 8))
 (segment (start 4 23.94) (end 4 16) (width 0.2) (layer "F.Cu") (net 26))
 (segment (start 4 16) (end 6.08 13.92) (width 0.2) (layer "F.Cu") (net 26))
 (segment (start 6.08 13.92) (end 6.78 13.92) (width 0.2) (layer "F.Cu") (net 26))
 (segment (start 0 27.94) (end 4 23.94) (width 0.2) (layer "F.Cu") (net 26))
 (segment (start 16.08 10.11) (end 17.83 10.11) (width 0.2) (layer "F.Cu") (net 12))
 (segment (start 17.83 10.11) (end 22.86 5.08) (width 0.2) (layer "F.Cu") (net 12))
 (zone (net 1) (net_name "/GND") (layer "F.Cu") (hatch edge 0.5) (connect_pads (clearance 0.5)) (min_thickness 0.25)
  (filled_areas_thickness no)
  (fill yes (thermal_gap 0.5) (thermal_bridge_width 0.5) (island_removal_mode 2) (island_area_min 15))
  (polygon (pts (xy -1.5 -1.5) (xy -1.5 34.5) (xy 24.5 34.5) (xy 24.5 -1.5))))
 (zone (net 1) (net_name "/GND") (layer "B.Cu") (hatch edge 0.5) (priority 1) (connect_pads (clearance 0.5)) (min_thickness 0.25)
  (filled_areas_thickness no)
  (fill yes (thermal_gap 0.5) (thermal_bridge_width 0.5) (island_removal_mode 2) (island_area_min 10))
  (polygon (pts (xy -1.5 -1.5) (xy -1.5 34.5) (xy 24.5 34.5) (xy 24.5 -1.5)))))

